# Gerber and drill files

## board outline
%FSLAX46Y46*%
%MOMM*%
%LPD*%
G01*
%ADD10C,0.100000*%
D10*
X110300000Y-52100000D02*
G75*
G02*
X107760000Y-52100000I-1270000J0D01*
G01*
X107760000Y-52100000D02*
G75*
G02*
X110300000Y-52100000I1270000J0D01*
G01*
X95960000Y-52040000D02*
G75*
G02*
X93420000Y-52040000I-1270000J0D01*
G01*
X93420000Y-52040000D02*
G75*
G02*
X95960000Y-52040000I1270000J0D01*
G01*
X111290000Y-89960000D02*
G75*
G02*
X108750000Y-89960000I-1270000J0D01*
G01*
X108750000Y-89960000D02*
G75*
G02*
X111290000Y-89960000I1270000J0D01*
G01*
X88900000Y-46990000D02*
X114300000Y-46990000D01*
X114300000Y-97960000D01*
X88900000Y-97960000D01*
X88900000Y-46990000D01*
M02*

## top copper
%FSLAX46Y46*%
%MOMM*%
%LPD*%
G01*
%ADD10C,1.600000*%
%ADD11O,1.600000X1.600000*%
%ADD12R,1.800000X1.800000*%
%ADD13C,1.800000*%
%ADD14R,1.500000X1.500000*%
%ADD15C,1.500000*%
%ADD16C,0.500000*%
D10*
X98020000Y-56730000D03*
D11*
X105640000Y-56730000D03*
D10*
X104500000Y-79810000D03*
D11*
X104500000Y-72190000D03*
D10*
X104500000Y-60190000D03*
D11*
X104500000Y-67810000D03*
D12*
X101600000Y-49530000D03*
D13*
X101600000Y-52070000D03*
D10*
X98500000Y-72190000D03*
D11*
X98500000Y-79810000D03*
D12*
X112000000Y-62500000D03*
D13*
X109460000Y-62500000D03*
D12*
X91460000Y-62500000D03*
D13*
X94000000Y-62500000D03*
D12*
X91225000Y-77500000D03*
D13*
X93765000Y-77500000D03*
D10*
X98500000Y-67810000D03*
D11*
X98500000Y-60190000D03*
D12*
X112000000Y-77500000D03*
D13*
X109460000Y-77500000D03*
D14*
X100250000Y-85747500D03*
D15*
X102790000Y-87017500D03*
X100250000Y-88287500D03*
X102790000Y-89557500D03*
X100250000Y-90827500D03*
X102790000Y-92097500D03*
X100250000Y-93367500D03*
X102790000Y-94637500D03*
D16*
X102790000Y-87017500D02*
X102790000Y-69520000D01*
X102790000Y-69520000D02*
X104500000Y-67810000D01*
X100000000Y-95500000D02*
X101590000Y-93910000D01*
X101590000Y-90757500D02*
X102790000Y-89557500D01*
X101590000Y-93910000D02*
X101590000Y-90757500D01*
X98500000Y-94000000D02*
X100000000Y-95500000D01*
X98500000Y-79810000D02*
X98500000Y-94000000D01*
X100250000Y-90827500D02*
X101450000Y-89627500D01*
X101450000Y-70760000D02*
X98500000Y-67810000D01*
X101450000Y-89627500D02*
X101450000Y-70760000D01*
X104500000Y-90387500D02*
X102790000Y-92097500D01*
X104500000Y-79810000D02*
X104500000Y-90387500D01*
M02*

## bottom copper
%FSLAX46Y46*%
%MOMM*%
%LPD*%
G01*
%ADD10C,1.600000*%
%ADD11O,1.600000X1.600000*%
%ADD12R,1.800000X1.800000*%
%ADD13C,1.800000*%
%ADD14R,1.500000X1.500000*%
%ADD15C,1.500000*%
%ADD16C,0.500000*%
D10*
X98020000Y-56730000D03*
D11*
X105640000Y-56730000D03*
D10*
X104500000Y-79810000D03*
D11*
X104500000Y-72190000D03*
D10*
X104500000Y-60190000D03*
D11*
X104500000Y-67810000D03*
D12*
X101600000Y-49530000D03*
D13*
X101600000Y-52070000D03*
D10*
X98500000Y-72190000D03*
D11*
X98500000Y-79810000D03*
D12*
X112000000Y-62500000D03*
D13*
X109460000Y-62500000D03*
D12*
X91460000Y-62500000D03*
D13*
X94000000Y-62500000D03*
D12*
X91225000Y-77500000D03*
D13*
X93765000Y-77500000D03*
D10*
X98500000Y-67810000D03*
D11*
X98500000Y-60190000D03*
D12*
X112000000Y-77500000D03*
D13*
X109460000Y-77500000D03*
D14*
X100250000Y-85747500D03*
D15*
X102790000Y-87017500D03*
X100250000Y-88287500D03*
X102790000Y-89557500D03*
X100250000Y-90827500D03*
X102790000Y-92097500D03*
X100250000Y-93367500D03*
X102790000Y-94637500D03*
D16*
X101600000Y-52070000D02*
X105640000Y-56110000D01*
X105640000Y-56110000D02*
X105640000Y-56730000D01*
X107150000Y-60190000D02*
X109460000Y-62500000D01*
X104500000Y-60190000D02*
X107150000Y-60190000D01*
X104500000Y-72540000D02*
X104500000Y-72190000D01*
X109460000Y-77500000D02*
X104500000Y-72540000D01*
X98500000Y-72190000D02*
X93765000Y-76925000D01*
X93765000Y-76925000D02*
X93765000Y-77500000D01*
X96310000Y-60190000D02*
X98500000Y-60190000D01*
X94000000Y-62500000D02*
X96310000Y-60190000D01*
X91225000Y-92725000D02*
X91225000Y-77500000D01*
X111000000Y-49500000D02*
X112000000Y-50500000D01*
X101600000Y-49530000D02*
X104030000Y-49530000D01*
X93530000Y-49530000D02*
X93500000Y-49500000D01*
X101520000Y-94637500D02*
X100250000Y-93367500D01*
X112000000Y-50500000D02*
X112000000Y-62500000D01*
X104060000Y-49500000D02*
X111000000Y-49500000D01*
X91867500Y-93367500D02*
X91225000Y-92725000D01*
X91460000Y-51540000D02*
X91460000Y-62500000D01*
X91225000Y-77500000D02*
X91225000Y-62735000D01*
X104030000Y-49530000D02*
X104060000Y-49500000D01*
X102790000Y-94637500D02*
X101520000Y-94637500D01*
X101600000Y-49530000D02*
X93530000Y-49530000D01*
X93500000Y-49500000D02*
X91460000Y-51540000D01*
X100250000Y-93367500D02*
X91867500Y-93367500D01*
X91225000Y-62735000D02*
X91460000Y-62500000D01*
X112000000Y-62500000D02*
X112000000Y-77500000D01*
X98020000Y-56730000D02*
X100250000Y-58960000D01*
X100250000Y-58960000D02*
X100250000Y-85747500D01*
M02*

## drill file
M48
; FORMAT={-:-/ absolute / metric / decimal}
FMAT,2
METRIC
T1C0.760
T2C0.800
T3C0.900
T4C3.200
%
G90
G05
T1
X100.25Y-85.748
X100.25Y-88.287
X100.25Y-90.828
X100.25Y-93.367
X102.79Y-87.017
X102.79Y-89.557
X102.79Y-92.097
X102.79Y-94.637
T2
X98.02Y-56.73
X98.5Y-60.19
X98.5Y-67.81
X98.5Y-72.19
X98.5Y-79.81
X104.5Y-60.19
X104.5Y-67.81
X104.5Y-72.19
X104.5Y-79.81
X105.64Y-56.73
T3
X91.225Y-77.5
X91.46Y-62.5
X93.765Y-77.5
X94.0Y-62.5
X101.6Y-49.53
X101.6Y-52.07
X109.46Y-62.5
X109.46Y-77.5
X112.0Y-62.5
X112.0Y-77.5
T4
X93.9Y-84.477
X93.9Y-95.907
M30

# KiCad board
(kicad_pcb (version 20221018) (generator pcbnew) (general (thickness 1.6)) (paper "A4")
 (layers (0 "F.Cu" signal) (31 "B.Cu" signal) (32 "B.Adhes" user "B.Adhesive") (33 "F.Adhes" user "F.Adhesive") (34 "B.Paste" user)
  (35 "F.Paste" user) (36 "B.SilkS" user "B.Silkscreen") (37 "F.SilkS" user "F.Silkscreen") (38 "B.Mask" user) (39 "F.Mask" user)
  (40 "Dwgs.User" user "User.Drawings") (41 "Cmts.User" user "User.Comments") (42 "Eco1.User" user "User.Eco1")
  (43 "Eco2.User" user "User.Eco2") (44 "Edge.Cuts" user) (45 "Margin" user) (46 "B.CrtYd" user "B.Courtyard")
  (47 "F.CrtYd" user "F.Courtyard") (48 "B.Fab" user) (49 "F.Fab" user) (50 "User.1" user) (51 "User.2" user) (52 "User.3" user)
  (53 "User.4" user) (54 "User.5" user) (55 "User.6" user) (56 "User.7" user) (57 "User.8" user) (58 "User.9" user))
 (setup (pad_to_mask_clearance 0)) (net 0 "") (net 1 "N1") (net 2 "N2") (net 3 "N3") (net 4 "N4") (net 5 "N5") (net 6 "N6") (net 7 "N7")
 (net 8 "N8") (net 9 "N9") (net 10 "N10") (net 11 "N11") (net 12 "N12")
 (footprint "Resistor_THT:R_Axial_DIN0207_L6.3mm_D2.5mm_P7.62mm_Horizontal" (layer "F.Cu") (at 98.02 56.73)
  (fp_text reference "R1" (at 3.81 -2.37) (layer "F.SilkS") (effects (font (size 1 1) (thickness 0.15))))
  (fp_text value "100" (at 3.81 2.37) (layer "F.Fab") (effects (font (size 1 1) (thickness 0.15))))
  (pad "1" thru_hole circle (at 0 0) (size 1.6 1.6) (drill 0.8) (layers "*.Cu" "*.Mask") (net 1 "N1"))
  (pad "2" thru_hole oval (at 7.62 0) (size 1.6 1.6) (drill 0.8) (layers "*.Cu" "*.Mask") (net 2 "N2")))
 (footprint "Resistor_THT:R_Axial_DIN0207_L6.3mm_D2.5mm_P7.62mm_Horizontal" (layer "F.Cu") (at 104.5 79.81 90)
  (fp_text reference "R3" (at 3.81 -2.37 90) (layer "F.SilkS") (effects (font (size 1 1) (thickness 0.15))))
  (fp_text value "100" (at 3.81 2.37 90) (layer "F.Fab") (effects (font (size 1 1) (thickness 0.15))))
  (pad "1" thru_hole circle (at 0 0 90) (size 1.6 1.6) (drill 0.8) (layers "*.Cu" "*.Mask") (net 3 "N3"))
  (pad "2" thru_hole oval (at 7.62 0 90) (size 1.6 1.6) (drill 0.8) (layers "*.Cu" "*.Mask") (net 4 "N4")))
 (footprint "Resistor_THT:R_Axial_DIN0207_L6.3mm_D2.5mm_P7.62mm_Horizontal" (layer "F.Cu") (at 104.5 60.19 -90)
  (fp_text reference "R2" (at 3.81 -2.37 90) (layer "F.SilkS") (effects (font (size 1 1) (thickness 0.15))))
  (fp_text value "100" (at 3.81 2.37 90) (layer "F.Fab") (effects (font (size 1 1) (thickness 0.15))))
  (pad "1" thru_hole circle (at 0 0 270) (size 1.6 1.6) (drill 0.8) (layers "*.Cu" "*.Mask") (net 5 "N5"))
  (pad "2" thru_hole oval (at 7.62 0 270) (size 1.6 1.6) (drill 0.8) (layers "*.Cu" "*.Mask") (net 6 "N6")))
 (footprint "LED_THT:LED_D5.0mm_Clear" (layer "F.Cu") (at 101.6 49.53 -90)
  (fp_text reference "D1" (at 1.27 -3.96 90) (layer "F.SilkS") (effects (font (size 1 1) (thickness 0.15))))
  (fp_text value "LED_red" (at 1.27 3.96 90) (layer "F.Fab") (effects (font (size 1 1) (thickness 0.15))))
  (pad "1" thru_hole rect (at 0 0 270) (size 1.8 1.8) (drill 0.9) (layers "*.Cu" "*.Mask") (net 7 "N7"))
  (pad "2" thru_hole circle (at 2.54 0 270) (size 1.8 1.8) (drill 0.9) (layers "*.Cu" "*.Mask") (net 2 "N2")))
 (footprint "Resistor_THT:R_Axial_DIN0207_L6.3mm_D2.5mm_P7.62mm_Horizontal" (layer "F.Cu") (at 98.5 72.19 -90)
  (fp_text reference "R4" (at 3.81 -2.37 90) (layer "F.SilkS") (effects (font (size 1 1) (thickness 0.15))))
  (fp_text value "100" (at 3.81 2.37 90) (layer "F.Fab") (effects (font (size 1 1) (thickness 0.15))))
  (pad "1" thru_hole circle (at 0 0 270) (size 1.6 1.6) (drill 0.8) (layers "*.Cu" "*.Mask") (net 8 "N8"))
  (pad "2" thru_hole oval (at 7.62 0 270) (size 1.6 1.6) (drill 0.8) (layers "*.Cu" "*.Mask") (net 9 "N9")))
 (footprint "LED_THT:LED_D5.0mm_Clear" (layer "F.Cu") (at 112 62.5 180)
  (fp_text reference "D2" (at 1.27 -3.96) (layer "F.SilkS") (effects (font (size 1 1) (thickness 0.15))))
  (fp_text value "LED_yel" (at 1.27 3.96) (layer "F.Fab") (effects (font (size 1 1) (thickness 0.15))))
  (pad "1" thru_hole rect (at 0 0 180) (size 1.8 1.8) (drill 0.9) (layers "*.Cu" "*.Mask") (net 7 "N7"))
  (pad "2" thru_hole circle (at 2.54 0 180) (size 1.8 1.8) (drill 0.9) (layers "*.Cu" "*.Mask") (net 5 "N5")))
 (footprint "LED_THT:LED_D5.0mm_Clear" (layer "F.Cu") (at 91.46 62.5)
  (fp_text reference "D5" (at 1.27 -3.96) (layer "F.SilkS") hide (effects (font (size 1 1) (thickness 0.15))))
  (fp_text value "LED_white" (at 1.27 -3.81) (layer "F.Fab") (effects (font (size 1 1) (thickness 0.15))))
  (pad "1" thru_hole rect (at 0 0) (size 1.8 1.8) (drill 0.9) (layers "*.Cu" "*.Mask") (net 7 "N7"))
  (pad "2" thru_hole circle (at 2.54 0) (size 1.8 1.8) (drill 0.9) (layers "*.Cu" "*.Mask") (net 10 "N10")))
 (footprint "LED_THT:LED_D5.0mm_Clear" (layer "F.Cu") (at 91.225 77.5)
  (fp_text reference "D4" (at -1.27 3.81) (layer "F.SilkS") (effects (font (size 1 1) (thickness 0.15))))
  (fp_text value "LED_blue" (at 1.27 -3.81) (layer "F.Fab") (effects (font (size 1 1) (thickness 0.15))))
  (pad "1" thru_hole rect (at 0 0) (size 1.8 1.8) (drill 0.9) (layers "*.Cu" "*.Mask") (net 7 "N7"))
  (pad "2" thru_hole circle (at 2.54 0) (size 1.8 1.8) (drill 0.9) (layers "*.Cu" "*.Mask") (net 8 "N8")))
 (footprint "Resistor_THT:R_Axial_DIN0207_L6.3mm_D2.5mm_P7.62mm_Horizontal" (layer "F.Cu") (at 98.5 67.81 90)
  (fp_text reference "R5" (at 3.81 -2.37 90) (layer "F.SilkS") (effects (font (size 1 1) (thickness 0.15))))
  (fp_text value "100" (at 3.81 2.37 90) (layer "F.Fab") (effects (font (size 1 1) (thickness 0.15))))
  (pad "1" thru_hole circle (at 0 0 90) (size 1.6 1.6) (drill 0.8) (layers "*.Cu" "*.Mask") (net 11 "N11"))
  (pad "2" thru_hole oval (at 7.62 0 90) (size 1.6 1.6) (drill 0.8) (layers "*.Cu" "*.Mask") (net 10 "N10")))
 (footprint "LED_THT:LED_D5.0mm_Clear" (layer "F.Cu") (at 112 77.5 180)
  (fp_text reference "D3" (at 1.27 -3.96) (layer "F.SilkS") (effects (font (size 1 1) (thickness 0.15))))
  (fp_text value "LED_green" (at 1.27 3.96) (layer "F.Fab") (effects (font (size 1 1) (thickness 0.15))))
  (pad "1" thru_hole rect (at 0 0 180) (size 1.8 1.8) (drill 0.9) (layers "*.Cu" "*.Mask") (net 7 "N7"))
  (pad "2" thru_hole circle (at 2.54 0 180) (size 1.8 1.8) (drill 0.9) (layers "*.Cu" "*.Mask") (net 4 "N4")))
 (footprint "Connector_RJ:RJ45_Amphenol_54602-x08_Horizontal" (layer "F.Cu") (at 100.25 85.7475 -90)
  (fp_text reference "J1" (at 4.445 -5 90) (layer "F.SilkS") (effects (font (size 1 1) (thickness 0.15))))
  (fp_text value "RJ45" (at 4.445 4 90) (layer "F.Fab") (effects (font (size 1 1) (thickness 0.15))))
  (pad "" np_thru_hole circle (at -1.27 6.35 270) (size 3.2 3.2) (drill 3.2) (layers "*.Cu" "*.Mask"))
  (pad "" np_thru_hole circle (at 10.16 6.35 270) (size 3.2 3.2) (drill 3.2) (layers "*.Cu" "*.Mask"))
  (pad "1" thru_hole rect (at 0 0 270) (size 1.5 1.5) (drill 0.76) (layers "*.Cu" "*.Mask") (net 1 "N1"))
  (pad "2" thru_hole circle (at 1.27 -2.54 270) (size 1.5 1.5) (drill 0.76) (layers "*.Cu" "*.Mask") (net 6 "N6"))
  (pad "3" thru_hole circle (at 2.54 0 270) (size 1.5 1.5) (drill 0.76) (layers "*.Cu" "*.Mask") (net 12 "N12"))
  (pad "4" thru_hole circle (at 3.81 -2.54 270) (size 1.5 1.5) (drill 0.76) (layers "*.Cu" "*.Mask") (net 9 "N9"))
  (pad "5" thru_hole circle (at 5.08 0 270) (size 1.5 1.5) (drill 0.76) (layers "*.Cu" "*.Mask") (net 11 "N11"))
  (pad "6" thru_hole circle (at 6.35 -2.54 270) (size 1.5 1.5) (drill 0.76) (layers "*.Cu" "*.Mask") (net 3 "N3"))
  (pad "7" thru_hole circle (at 7.62 0 270) (size 1.5 1.5) (drill 0.76) (layers "*.Cu" "*.Mask") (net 7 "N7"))
  (pad "8" thru_hole circle (at 8.89 -2.54 270) (size 1.5 1.5) (drill 0.76) (layers "*.Cu" "*.Mask") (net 7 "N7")))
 (gr_circle (center 109.03 52.1) (end 110.3 52.1) (stroke (width 0.1) (type default)) (fill none) (layer "Edge.Cuts"))
 (gr_circle (center 94.69 52.04) (end 93.42 52.04) (stroke (width 0.1) (type default)) (fill none) (layer "Edge.Cuts"))
 (gr_circle (center 110.02 89.96) (end 108.75 89.96) (stroke (width 0.1) (type default)) (fill none) (layer "Edge.Cuts"))
 (gr_rect (start 88.9 46.99) (end 114.3 97.96) (stroke (width 0.1) (type default)) (fill none) (layer "Edge.Cuts"))
 (segment (start 101.6 52.07) (end 105.64 56.11) (width 0.5) (layer "B.Cu") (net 2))
 (segment (start 105.64 56.11) (end 105.64 56.73) (width 0.5) (layer "B.Cu") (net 2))
 (segment (start 107.15 60.19) (end 109.46 62.5) (width 0.5) (layer "B.Cu") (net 5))
 (segment (start 104.5 60.19) (end 107.15 60.19) (width 0.5) (layer "B.Cu") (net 5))
 (segment (start 104.5 72.54) (end 104.5 72.19) (width 0.5) (layer "B.Cu") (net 4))
 (segment (start 109.46 77.5) (end 104.5 72.54) (width 0.5) (layer "B.Cu") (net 4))
 (segment (start 98.5 72.19) (end 93.765 76.925) (width 0.5) (layer "B.Cu") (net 8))
 (segment (start 93.765 76.925) (end 93.765 77.5) (width 0.5) (layer "B.Cu") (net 8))
 (segment (start 96.31 60.19) (end 98.5 60.19) (width 0.5) (layer "B.Cu") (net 10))
 (segment (start 94 62.5) (end 96.31 60.19) (width 0.5) (layer "B.Cu") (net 10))
 (segment (start 91.225 92.725) (end 91.225 77.5) (width 0.5) (layer "B.Cu") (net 7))
 (segment (start 111 49.5) (end 112 50.5) (width 0.5) (layer "B.Cu") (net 7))
 (segment (start 101.6 49.53) (end 104.03 49.53) (width 0.5) (layer "B.Cu") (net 7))
 (segment (start 93.53 49.53) (end 93.5 49.5) (width 0.5) (layer "B.Cu") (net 7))
 (segment (start 101.52 94.6375) (end 100.25 93.3675) (width 0.5) (layer "B.Cu") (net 7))
 (segment (start 112 50.5) (end 112 62.5) (width 0.5) (layer "B.Cu") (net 7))
 (segment (start 104.06 49.5) (end 111 49.5) (width 0.5) (layer "B.Cu") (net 7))
 (segment (start 91.8675 93.3675) (end 91.225 92.725) (width 0.5) (layer "B.Cu") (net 7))
 (segment (start 91.46 51.54) (end 91.46 62.5) (width 0.5) (layer "B.Cu") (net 7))
 (segment (start 91.225 77.5) (end 91.225 62.735) (width 0.5) (layer "B.Cu") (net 7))
 (segment (start 104.03 49.53) (end 104.06 49.5) (width 0.5) (layer "B.Cu") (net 7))
 (segment (start 102.79 94.6375) (end 101.52 94.6375) (width 0.5) (layer "B.Cu") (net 7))
 (segment (start 101.6 49.53) (end 93.53 49.53) (width 0.5) (layer "B.Cu") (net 7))
 (segment (start 93.5 49.5) (end 91.46 51.54) (width 0.5) (layer "B.Cu") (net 7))
 (segment (start 100.25 93.3675) (end 91.8675 93.3675) (width 0.5) (layer "B.Cu") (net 7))
 (segment (start 91.225 62.735) (end 91.46 62.5) (width 0.5) (layer "B.Cu") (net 7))
 (segment (start 112 62.5) (end 112 77.5) (width 0.5) (layer "B.Cu") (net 7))
 (segment (start 98.02 56.73) (end 100.25 58.96) (width 0.5) (layer "B.Cu") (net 1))
 (segment (start 100.25 58.96) (end 100.25 85.7475) (width 0.5) (layer "B.Cu") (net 1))
 (segment (start 102.79 87.0175) (end 102.79 69.52) (width 0.5) (layer "F.Cu") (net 6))
 (segment (start 102.79 69.52) (end 104.5 67.81) (width 0.5) (layer "F.Cu") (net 6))
 (segment (start 100 95.5) (end 101.59 93.91) (width 0.5) (layer "F.Cu") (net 9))
 (segment (start 101.59 90.7575) (end 102.79 89.5575) (width 0.5) (layer "F.Cu") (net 9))
 (segment (start 101.59 93.91) (end 101.59 90.7575) (width 0.5) (layer "F.Cu") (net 9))
 (segment (start 98.5 94) (end 100 95.5) (width 0.5) (layer "F.Cu") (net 9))
 (segment (start 98.5 79.81) (end 98.5 94) (width 0.5) (layer "F.Cu") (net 9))
 (segment (start 100.25 90.8275) (end 101.45 89.6275) (width 0.5) (layer "F.Cu") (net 11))
 (segment (start 101.45 70.76) (end 98.5 67.81) (width 0.5) (layer "F.Cu") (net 11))
 (segment (start 101.45 89.6275) (end 101.45 70.76) (width 0.5) (layer "F.Cu") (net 11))
 (segment (start 104.5 90.3875) (end 102.79 92.0975) (width 0.5) (layer "F.Cu") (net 3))
 (segment (start 104.5 79.81) (end 104.5 90.3875) (width 0.5) (layer "F.Cu") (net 3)))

